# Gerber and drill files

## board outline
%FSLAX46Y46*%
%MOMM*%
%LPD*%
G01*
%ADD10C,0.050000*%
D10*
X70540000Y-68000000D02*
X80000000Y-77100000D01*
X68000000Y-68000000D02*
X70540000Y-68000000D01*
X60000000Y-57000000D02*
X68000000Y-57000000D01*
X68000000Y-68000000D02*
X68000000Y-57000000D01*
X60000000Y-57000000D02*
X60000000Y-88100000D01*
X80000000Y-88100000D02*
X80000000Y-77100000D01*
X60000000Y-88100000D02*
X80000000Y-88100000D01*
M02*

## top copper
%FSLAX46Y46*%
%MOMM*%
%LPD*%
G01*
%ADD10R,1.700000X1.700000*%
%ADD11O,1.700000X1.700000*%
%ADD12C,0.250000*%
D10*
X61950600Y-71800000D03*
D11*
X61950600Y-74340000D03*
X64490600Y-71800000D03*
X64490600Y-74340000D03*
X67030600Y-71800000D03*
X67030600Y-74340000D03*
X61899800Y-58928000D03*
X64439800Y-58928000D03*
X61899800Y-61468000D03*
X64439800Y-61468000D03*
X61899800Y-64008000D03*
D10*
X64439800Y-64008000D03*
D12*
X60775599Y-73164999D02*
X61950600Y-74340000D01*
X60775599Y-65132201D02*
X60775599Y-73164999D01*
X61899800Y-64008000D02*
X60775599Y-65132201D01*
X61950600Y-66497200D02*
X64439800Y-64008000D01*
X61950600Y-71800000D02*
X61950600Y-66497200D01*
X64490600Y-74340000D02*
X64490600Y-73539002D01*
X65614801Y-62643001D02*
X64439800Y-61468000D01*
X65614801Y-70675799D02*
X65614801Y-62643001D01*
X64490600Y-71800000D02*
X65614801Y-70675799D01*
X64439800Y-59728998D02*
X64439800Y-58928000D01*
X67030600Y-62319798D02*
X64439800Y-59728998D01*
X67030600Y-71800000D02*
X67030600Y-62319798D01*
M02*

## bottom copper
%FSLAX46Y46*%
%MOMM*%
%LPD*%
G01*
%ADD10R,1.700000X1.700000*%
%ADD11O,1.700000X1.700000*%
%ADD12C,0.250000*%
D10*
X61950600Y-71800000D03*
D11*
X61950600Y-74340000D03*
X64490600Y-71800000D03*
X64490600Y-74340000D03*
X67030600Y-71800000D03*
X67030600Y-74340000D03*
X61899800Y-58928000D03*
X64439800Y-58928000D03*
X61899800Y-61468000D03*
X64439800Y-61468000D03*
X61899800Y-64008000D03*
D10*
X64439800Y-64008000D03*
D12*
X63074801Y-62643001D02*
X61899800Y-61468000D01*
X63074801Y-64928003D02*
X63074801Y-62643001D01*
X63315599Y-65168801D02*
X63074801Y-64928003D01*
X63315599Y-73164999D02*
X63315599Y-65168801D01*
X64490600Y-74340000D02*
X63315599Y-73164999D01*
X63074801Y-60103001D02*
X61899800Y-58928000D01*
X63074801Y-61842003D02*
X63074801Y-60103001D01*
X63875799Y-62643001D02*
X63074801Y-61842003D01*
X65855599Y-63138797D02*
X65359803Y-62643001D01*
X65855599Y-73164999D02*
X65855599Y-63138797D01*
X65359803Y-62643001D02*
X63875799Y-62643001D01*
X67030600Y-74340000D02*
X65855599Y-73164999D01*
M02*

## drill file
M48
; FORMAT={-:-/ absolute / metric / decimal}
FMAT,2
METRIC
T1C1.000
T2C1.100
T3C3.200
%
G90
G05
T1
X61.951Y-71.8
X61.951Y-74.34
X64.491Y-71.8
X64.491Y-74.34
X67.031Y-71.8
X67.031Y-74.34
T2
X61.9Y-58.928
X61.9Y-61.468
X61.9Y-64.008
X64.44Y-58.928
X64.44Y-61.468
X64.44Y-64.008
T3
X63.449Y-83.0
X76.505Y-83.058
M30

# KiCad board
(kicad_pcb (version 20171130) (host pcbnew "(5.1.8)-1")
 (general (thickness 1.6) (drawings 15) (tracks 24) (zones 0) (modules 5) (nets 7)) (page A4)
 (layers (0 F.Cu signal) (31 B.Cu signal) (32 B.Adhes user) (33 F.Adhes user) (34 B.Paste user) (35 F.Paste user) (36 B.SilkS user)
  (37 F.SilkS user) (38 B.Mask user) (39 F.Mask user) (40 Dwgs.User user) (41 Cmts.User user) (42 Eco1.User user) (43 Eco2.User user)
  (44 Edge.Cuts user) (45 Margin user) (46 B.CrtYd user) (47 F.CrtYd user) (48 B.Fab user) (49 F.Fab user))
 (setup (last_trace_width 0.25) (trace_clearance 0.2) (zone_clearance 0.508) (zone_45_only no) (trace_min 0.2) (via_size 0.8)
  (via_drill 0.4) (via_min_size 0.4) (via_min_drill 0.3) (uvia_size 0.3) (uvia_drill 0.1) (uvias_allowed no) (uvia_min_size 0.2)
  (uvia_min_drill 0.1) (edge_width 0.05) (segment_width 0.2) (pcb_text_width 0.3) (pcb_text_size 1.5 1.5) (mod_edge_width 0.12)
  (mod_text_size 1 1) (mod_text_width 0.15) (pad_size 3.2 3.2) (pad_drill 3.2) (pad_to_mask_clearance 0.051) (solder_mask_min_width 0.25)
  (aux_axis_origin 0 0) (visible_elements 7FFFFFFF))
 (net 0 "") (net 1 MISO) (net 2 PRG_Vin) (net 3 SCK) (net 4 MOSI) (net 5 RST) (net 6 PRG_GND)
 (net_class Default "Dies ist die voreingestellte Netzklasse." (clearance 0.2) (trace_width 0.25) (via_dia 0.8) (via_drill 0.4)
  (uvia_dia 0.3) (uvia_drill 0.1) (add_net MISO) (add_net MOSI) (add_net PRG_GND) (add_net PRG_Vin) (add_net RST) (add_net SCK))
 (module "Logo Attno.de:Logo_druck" (layer F.Cu) (at 69.9262 81.6864)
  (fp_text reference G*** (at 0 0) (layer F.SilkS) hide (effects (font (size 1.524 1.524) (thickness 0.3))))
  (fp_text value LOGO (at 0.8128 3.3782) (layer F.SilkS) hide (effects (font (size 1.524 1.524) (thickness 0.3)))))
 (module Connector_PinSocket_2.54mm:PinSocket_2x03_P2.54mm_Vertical (layer F.Cu) (at 61.9506 71.8 90)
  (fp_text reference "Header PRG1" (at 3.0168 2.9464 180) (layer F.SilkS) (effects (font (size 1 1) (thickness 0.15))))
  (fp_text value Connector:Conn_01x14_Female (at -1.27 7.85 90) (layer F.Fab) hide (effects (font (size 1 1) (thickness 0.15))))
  (pad 1 thru_hole rect (at 0 0 90) (size 1.7 1.7) (drill 1) (layers *.Cu *.Mask) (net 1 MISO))
  (pad 2 thru_hole oval (at -2.54 0 90) (size 1.7 1.7) (drill 1) (layers *.Cu *.Mask) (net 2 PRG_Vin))
  (pad 3 thru_hole oval (at 0 2.54 90) (size 1.7 1.7) (drill 1) (layers *.Cu *.Mask) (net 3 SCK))
  (pad 4 thru_hole oval (at -2.54 2.54 90) (size 1.7 1.7) (drill 1) (layers *.Cu *.Mask) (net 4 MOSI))
  (pad 5 thru_hole oval (at 0 5.08 90) (size 1.7 1.7) (drill 1) (layers *.Cu *.Mask) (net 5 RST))
  (pad 6 thru_hole oval (at -2.54 5.08 90) (size 1.7 1.7) (drill 1) (layers *.Cu *.Mask) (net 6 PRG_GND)))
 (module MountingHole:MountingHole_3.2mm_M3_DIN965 (layer F.Cu) (at 76.5048 83.058)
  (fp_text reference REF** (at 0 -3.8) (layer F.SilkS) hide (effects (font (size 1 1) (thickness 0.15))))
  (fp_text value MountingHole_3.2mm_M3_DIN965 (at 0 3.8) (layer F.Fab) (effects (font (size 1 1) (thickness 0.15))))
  (pad 1 np_thru_hole circle (at 0 0) (size 3.2 3.2) (drill 3.2) (layers *.Cu *.Mask)))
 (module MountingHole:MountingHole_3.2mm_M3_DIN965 (layer F.Cu) (at 63.4492 83)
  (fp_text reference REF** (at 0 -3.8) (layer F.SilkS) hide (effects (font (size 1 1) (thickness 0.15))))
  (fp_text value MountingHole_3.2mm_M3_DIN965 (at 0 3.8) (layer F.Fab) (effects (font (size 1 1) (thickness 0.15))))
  (pad 1 np_thru_hole circle (at 0 0) (size 3.2 3.2) (drill 3.2) (layers *.Cu *.Mask)))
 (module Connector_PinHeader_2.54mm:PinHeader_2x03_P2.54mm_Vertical (layer F.Cu) (at 64.4398 64.008 180)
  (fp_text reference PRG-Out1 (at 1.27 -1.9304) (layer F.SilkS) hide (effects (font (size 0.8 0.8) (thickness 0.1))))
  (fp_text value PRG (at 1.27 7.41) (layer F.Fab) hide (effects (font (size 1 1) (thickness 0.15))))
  (pad 6 thru_hole oval (at 2.54 5.08 180) (size 1.7 1.7) (drill 1.1) (layers *.Cu *.Mask) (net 6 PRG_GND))
  (pad 5 thru_hole oval (at 0 5.08 180) (size 1.7 1.7) (drill 1.1) (layers *.Cu *.Mask) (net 5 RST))
  (pad 4 thru_hole oval (at 2.54 2.54 180) (size 1.7 1.7) (drill 1.1) (layers *.Cu *.Mask) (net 4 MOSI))
  (pad 3 thru_hole oval (at 0 2.54 180) (size 1.7 1.7) (drill 1.1) (layers *.Cu *.Mask) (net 3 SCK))
  (pad 2 thru_hole oval (at 2.54 0 180) (size 1.7 1.7) (drill 1.1) (layers *.Cu *.Mask) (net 2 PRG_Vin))
  (pad 1 thru_hole rect (at 0 0 180) (size 1.7 1.7) (drill 1.1) (layers *.Cu *.Mask) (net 1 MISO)))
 (gr_line (start 70.54 68) (end 80 77.1) (layer Edge.Cuts) (width 0.05))
 (gr_line (start 68 68) (end 70.54 68) (layer Edge.Cuts) (width 0.05))
 (gr_line (start 60 57) (end 68 57) (layer Edge.Cuts) (width 0.05))
 (gr_line (start 68 68) (end 68 57) (layer Edge.Cuts) (width 0.05))
 (gr_line (start 60 57) (end 60 88.1) (layer Edge.Cuts) (width 0.05))
 (gr_line (start 80 88.1) (end 80 77.1) (layer Edge.Cuts) (width 0.05))
 (gr_line (start 60 88.1) (end 80 88.1) (layer Edge.Cuts) (width 0.05))
 (segment (start 60.775599 73.164999) (end 61.9506 74.34) (width 0.25) (layer F.Cu) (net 2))
 (segment (start 60.775599 65.132201) (end 60.775599 73.164999) (width 0.25) (layer F.Cu) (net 2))
 (segment (start 61.8998 64.008) (end 60.775599 65.132201) (width 0.25) (layer F.Cu) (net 2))
 (segment (start 61.9506 66.4972) (end 64.4398 64.008) (width 0.25) (layer F.Cu) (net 1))
 (segment (start 61.9506 71.8) (end 61.9506 66.4972) (width 0.25) (layer F.Cu) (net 1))
 (segment (start 64.4906 74.34) (end 64.4906 73.539002) (width 0.25) (layer F.Cu) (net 4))
 (segment (start 63.074801 62.643001) (end 61.8998 61.468) (width 0.25) (layer B.Cu) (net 4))
 (segment (start 63.074801 64.928003) (end 63.074801 62.643001) (width 0.25) (layer B.Cu) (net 4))
 (segment (start 63.315599 65.168801) (end 63.074801 64.928003) (width 0.25) (layer B.Cu) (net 4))
 (segment (start 63.315599 73.164999) (end 63.315599 65.168801) (width 0.25) (layer B.Cu) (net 4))
 (segment (start 64.4906 74.34) (end 63.315599 73.164999) (width 0.25) (layer B.Cu) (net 4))
 (segment (start 65.614801 62.643001) (end 64.4398 61.468) (width 0.25) (layer F.Cu) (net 3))
 (segment (start 65.614801 70.675799) (end 65.614801 62.643001) (width 0.25) (layer F.Cu) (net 3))
 (segment (start 64.4906 71.8) (end 65.614801 70.675799) (width 0.25) (layer F.Cu) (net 3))
 (segment (start 64.4398 59.728998) (end 64.4398 58.928) (width 0.25) (layer F.Cu) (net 5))
 (segment (start 67.0306 62.319798) (end 64.4398 59.728998) (width 0.25) (layer F.Cu) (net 5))
 (segment (start 67.0306 71.8) (end 67.0306 62.319798) (width 0.25) (layer F.Cu) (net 5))
 (segment (start 63.074801 60.103001) (end 61.8998 58.928) (width 0.25) (layer B.Cu) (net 6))
 (segment (start 63.074801 61.842003) (end 63.074801 60.103001) (width 0.25) (layer B.Cu) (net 6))
 (segment (start 63.875799 62.643001) (end 63.074801 61.842003) (width 0.25) (layer B.Cu) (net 6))
 (segment (start 65.855599 63.138797) (end 65.359803 62.643001) (width 0.25) (layer B.Cu) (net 6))
 (segment (start 65.855599 73.164999) (end 65.855599 63.138797) (width 0.25) (layer B.Cu) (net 6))
 (segment (start 65.359803 62.643001) (end 63.875799 62.643001) (width 0.25) (layer B.Cu) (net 6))
 (segment (start 67.0306 74.34) (end 65.855599 73.164999) (width 0.25) (layer B.Cu) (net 6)))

